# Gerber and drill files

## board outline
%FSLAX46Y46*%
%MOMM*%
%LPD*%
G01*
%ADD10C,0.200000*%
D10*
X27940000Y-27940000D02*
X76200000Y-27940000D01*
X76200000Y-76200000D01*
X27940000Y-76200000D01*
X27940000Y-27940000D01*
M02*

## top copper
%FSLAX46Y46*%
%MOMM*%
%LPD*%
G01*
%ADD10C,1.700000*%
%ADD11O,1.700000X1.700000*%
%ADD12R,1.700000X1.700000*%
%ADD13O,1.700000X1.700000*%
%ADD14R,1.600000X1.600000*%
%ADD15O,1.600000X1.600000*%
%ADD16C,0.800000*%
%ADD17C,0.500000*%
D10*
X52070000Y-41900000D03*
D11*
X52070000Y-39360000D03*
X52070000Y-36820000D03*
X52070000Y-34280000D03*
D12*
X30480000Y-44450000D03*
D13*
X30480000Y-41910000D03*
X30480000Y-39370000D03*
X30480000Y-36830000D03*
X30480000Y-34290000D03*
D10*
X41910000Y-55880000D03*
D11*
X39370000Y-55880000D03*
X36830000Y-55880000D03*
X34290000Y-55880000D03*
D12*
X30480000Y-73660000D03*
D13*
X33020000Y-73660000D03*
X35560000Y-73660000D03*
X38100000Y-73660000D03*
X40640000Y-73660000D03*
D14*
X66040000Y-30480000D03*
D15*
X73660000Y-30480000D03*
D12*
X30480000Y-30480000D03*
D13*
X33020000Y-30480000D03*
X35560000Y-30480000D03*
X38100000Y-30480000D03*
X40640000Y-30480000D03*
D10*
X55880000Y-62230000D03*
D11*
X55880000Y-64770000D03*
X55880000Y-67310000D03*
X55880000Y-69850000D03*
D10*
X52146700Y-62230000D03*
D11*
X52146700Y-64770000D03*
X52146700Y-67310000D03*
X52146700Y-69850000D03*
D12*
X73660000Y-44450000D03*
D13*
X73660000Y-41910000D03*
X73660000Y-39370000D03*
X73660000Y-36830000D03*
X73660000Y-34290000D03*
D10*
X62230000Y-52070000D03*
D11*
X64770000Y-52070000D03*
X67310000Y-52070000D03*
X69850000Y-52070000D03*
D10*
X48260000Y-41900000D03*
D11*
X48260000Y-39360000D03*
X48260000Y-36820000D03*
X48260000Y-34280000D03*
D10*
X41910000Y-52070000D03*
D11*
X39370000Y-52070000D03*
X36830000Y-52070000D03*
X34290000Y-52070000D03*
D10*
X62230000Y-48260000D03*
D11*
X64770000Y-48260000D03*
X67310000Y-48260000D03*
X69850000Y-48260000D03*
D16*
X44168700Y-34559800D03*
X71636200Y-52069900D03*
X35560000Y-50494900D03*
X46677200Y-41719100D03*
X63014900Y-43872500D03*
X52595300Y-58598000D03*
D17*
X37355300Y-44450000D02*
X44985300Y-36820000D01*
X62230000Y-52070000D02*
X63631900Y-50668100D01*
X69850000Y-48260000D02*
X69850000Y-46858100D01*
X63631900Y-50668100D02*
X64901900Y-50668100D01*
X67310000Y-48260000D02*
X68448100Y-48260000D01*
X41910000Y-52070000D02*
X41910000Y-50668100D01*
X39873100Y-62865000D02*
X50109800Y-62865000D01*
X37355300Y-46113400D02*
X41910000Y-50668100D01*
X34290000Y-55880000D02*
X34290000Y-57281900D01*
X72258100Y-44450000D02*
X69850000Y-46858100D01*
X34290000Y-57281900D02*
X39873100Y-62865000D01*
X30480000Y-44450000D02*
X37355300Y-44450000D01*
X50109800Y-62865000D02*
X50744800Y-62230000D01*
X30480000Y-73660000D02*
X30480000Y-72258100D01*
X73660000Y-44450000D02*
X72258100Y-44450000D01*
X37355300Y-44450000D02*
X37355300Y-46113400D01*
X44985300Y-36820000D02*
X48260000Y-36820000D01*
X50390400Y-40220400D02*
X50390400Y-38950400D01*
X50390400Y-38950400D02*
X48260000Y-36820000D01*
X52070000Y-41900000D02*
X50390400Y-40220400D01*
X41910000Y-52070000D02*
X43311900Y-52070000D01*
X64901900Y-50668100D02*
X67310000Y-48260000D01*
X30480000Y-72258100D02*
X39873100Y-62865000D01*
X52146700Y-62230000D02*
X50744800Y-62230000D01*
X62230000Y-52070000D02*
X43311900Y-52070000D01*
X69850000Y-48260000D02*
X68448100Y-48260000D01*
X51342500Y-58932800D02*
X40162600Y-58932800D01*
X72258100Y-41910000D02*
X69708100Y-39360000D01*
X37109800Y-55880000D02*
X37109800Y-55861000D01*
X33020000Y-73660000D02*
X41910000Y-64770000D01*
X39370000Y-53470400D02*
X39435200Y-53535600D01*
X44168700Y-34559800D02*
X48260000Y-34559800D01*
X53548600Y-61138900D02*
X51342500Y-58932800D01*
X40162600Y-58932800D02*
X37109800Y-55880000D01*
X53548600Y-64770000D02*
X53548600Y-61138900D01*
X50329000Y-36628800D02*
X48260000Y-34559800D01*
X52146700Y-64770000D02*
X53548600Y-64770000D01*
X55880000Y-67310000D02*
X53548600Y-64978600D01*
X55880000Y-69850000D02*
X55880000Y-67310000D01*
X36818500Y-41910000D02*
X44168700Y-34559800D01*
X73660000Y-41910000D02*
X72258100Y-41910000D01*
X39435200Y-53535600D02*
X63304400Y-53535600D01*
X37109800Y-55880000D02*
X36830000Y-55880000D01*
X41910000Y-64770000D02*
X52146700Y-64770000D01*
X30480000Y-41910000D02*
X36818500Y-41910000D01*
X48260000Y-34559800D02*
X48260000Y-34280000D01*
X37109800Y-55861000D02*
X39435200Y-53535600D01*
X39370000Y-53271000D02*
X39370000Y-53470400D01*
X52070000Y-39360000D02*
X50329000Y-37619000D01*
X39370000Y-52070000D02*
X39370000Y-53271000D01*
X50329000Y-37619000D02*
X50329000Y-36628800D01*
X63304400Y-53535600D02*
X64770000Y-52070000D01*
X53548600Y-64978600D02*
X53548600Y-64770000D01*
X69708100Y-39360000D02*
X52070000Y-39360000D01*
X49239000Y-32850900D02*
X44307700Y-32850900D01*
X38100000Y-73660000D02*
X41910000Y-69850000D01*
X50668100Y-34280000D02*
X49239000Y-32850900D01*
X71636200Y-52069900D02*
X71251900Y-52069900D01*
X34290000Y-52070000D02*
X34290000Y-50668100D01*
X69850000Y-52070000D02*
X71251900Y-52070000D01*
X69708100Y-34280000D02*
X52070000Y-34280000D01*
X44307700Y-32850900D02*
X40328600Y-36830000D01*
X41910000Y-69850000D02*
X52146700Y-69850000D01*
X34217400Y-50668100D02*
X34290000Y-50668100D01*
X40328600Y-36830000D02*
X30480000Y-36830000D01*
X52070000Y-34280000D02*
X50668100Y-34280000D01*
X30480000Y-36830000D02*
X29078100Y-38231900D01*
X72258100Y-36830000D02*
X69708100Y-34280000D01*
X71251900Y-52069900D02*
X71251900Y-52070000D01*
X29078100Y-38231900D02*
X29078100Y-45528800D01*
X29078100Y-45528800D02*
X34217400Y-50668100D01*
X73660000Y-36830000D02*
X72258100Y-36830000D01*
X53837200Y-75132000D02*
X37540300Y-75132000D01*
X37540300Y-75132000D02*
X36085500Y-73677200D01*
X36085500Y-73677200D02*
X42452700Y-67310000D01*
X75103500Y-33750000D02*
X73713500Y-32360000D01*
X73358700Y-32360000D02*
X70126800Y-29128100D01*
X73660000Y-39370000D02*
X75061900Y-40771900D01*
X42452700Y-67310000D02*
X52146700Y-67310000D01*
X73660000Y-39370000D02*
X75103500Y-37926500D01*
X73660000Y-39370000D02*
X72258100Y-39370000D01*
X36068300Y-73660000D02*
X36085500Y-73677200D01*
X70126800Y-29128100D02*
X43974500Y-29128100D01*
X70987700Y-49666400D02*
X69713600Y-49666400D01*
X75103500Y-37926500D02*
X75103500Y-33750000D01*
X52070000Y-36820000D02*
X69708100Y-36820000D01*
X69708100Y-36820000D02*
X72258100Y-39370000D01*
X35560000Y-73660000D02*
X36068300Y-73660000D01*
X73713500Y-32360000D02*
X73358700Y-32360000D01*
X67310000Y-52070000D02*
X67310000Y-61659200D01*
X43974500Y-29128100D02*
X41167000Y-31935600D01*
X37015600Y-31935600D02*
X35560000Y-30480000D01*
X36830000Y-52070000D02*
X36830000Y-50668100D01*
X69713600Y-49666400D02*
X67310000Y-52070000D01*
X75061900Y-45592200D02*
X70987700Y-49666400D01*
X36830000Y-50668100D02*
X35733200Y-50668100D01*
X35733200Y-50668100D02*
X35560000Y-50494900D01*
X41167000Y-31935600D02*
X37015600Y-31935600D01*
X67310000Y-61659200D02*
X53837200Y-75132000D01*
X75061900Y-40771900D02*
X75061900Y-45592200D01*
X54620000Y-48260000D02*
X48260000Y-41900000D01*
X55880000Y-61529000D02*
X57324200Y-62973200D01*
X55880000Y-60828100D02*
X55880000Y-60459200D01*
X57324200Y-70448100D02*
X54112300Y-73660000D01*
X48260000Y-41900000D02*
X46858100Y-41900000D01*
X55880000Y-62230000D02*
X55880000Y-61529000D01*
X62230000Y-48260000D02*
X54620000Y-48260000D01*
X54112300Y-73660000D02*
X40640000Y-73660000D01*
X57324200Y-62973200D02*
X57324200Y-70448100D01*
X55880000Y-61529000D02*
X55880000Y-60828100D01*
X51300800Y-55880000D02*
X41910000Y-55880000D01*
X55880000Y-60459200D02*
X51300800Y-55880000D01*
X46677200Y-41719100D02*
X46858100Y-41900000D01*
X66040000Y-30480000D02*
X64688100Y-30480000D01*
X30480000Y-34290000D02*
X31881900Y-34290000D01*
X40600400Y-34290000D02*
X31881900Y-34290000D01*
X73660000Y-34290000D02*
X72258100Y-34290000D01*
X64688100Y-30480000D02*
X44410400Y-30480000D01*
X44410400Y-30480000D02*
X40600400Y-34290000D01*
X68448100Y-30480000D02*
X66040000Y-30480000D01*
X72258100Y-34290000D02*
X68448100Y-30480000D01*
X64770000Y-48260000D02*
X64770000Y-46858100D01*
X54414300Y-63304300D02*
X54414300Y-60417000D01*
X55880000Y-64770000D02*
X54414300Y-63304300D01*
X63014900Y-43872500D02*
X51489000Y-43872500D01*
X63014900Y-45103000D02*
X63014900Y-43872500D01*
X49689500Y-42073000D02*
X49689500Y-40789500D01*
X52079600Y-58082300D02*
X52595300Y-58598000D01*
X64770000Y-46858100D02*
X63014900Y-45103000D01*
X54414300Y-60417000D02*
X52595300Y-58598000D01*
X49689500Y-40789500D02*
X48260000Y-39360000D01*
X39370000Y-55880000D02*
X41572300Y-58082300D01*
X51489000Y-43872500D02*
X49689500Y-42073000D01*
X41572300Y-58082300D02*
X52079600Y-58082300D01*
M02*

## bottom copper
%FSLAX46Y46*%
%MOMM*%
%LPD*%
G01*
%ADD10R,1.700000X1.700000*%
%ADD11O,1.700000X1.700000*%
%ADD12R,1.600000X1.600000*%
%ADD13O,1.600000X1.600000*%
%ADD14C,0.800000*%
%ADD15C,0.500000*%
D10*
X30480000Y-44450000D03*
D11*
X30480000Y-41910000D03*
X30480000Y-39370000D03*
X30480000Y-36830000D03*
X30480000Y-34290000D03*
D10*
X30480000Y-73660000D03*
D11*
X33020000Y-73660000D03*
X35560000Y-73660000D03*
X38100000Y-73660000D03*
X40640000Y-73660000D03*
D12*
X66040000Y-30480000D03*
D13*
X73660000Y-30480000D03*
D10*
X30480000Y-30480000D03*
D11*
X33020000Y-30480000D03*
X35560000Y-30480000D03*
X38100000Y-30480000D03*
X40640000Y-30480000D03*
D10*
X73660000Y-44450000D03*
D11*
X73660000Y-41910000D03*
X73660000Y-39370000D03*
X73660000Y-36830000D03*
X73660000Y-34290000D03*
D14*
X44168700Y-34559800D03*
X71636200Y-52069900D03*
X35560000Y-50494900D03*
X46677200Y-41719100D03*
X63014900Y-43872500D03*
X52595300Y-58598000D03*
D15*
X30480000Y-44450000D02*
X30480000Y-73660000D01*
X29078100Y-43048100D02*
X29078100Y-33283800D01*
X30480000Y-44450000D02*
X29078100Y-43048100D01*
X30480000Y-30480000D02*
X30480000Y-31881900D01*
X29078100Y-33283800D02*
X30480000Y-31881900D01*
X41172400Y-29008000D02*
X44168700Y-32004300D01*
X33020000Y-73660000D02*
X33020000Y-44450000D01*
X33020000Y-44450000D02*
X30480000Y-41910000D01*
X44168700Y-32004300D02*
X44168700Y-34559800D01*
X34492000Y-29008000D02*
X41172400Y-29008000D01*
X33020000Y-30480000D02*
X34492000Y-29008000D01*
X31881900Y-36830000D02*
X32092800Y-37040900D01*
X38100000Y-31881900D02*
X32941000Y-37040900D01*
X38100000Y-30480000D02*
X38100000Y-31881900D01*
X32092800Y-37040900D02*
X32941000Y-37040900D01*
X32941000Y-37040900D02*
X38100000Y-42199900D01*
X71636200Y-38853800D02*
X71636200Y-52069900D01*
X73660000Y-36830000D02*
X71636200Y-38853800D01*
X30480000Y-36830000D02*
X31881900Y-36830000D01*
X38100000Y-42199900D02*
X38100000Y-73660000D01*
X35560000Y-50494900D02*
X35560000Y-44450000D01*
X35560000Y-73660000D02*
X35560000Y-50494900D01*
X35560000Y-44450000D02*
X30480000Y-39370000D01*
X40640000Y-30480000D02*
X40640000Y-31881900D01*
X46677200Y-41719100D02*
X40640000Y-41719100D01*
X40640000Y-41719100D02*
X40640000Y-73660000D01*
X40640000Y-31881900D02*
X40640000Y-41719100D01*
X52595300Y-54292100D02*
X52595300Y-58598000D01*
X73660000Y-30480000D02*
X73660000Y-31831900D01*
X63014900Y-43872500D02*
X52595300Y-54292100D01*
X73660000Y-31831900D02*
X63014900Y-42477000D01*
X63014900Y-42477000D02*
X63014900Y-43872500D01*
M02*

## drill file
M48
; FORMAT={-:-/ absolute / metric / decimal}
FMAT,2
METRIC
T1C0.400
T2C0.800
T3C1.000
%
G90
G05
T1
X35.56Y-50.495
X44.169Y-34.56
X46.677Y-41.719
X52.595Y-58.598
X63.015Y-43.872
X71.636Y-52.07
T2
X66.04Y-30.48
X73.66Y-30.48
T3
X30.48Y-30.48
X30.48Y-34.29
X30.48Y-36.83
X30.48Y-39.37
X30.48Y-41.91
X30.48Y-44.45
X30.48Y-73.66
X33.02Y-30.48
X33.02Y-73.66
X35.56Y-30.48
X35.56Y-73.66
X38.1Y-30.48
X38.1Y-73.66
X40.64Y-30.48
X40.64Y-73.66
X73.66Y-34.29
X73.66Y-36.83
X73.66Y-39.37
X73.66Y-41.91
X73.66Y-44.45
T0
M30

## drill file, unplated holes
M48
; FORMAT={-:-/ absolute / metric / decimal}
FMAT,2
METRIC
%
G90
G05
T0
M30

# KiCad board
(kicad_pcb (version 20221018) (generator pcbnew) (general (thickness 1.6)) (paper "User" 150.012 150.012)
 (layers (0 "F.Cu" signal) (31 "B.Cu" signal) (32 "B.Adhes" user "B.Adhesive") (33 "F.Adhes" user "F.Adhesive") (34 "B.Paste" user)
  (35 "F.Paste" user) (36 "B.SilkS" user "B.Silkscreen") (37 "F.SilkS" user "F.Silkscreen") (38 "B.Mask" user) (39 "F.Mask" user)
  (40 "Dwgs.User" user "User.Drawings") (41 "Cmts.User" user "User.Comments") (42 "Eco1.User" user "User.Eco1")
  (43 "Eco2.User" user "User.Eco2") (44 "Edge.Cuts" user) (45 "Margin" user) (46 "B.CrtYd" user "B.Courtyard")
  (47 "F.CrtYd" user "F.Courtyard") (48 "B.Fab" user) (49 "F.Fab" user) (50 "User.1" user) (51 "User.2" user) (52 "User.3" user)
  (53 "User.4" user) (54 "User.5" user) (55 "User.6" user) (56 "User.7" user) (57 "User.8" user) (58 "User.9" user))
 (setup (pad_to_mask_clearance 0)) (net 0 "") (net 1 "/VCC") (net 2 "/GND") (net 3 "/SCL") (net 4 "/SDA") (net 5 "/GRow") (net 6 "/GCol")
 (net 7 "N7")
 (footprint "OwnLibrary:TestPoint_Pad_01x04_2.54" (layer "F.Cu") (at 52.07 41.9 180)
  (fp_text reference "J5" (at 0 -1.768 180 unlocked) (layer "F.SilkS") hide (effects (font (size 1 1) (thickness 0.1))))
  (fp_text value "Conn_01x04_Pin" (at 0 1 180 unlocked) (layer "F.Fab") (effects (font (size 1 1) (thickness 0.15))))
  (pad "1" smd circle (at 0 0 180) (size 1.7 1.7) (layers "F.Cu" "F.Paste" "F.Mask") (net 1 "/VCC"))
  (pad "2" smd oval (at 0 2.54 180) (size 1.7 1.7) (layers "F.Cu" "F.Paste" "F.Mask") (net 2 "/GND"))
  (pad "3" smd oval (at 0 5.08 180) (size 1.7 1.7) (layers "F.Cu" "F.Paste" "F.Mask") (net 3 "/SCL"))
  (pad "4" smd oval (at 0 7.62 180) (size 1.7 1.7) (layers "F.Cu" "F.Paste" "F.Mask") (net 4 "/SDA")))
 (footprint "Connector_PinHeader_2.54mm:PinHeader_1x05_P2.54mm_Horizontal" (layer "F.Cu") (at 30.48 44.45 180)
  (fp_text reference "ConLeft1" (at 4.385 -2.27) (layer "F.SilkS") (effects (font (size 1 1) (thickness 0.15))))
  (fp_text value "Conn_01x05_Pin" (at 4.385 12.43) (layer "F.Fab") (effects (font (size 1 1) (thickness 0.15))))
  (pad "1" thru_hole rect (at 0 0 180) (size 1.7 1.7) (drill 1) (layers "*.Cu" "*.Mask") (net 1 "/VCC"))
  (pad "2" thru_hole oval (at 0 2.54 180) (size 1.7 1.7) (drill 1) (layers "*.Cu" "*.Mask") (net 2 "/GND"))
  (pad "3" thru_hole oval (at 0 5.08 180) (size 1.7 1.7) (drill 1) (layers "*.Cu" "*.Mask") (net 3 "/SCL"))
  (pad "4" thru_hole oval (at 0 7.62 180) (size 1.7 1.7) (drill 1) (layers "*.Cu" "*.Mask") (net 4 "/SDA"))
  (pad "5" thru_hole oval (at 0 10.16 180) (size 1.7 1.7) (drill 1) (layers "*.Cu" "*.Mask") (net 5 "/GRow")))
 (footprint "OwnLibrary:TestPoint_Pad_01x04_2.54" (layer "F.Cu") (at 41.91 55.88 -90)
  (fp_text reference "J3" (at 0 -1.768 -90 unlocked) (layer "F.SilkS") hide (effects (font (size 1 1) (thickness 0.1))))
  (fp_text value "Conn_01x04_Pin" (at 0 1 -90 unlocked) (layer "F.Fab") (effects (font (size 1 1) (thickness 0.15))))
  (pad "1" smd circle (at 0 0 270) (size 1.7 1.7) (layers "F.Cu" "F.Paste" "F.Mask") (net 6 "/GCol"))
  (pad "2" smd oval (at 0 2.54 270) (size 1.7 1.7) (layers "F.Cu" "F.Paste" "F.Mask") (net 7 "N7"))
  (pad "3" smd oval (at 0 5.08 270) (size 1.7 1.7) (layers "F.Cu" "F.Paste" "F.Mask") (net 2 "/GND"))
  (pad "4" smd oval (at 0 7.62 270) (size 1.7 1.7) (layers "F.Cu" "F.Paste" "F.Mask") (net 1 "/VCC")))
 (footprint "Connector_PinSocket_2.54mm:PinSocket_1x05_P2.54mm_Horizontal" (layer "F.Cu") (at 30.48 73.66 90)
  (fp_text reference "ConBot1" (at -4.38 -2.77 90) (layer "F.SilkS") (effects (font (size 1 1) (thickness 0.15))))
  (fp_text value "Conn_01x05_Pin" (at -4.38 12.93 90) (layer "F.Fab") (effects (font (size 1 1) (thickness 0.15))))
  (pad "1" thru_hole rect (at 0 0 90) (size 1.7 1.7) (drill 1) (layers "*.Cu" "*.Mask") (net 1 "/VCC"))
  (pad "2" thru_hole oval (at 0 2.54 90) (size 1.7 1.7) (drill 1) (layers "*.Cu" "*.Mask") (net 2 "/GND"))
  (pad "3" thru_hole oval (at 0 5.08 90) (size 1.7 1.7) (drill 1) (layers "*.Cu" "*.Mask") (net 3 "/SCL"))
  (pad "4" thru_hole oval (at 0 7.62 90) (size 1.7 1.7) (drill 1) (layers "*.Cu" "*.Mask") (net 4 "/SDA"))
  (pad "5" thru_hole oval (at 0 10.16 90) (size 1.7 1.7) (drill 1) (layers "*.Cu" "*.Mask") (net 6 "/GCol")))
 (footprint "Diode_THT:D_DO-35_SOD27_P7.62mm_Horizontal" (layer "F.Cu") (at 66.04 30.48)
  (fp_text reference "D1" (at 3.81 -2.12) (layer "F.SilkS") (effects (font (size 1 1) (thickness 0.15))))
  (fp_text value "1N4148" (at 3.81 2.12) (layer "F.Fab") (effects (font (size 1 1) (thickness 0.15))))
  (pad "1" thru_hole rect (at 0 0) (size 1.6 1.6) (drill 0.8) (layers "*.Cu" "*.Mask") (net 5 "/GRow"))
  (pad "2" thru_hole oval (at 7.62 0) (size 1.6 1.6) (drill 0.8) (layers "*.Cu" "*.Mask") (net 7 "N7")))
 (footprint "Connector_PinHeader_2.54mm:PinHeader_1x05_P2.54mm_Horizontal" (layer "F.Cu") (at 30.48 30.48 90)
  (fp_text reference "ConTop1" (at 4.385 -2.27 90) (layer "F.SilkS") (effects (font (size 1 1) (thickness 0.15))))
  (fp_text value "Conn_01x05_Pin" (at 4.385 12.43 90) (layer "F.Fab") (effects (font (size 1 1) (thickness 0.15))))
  (pad "1" thru_hole rect (at 0 0 90) (size 1.7 1.7) (drill 1) (layers "*.Cu" "*.Mask") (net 1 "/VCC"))
  (pad "2" thru_hole oval (at 0 2.54 90) (size 1.7 1.7) (drill 1) (layers "*.Cu" "*.Mask") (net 2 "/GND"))
  (pad "3" thru_hole oval (at 0 5.08 90) (size 1.7 1.7) (drill 1) (layers "*.Cu" "*.Mask") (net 3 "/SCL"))
  (pad "4" thru_hole oval (at 0 7.62 90) (size 1.7 1.7) (drill 1) (layers "*.Cu" "*.Mask") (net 4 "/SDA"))
  (pad "5" thru_hole oval (at 0 10.16 90) (size 1.7 1.7) (drill 1) (layers "*.Cu" "*.Mask") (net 6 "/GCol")))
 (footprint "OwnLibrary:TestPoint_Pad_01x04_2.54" (layer "F.Cu") (at 55.88 62.23)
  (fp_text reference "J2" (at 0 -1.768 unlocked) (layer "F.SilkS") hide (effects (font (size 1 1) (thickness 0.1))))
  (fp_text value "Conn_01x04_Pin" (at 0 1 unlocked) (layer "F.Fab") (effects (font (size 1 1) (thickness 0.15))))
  (pad "1" smd circle (at 0 0) (size 1.7 1.7) (layers "F.Cu" "F.Paste" "F.Mask") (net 6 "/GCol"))
  (pad "2" smd oval (at 0 2.54) (size 1.7 1.7) (layers "F.Cu" "F.Paste" "F.Mask") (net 7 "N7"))
  (pad "3" smd oval (at 0 5.08) (size 1.7 1.7) (layers "F.Cu" "F.Paste" "F.Mask") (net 2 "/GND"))
  (pad "4" smd oval (at 0 7.62) (size 1.7 1.7) (layers "F.Cu" "F.Paste" "F.Mask") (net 2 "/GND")))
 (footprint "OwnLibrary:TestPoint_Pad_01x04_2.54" (layer "F.Cu") (at 52.1467 62.23)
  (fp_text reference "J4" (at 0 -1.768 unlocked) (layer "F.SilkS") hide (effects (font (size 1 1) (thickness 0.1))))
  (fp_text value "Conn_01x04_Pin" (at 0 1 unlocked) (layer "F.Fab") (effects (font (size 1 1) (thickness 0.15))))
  (pad "1" smd circle (at 0 0) (size 1.7 1.7) (layers "F.Cu" "F.Paste" "F.Mask") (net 1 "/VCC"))
  (pad "2" smd oval (at 0 2.54) (size 1.7 1.7) (layers "F.Cu" "F.Paste" "F.Mask") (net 2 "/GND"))
  (pad "3" smd oval (at 0 5.08) (size 1.7 1.7) (layers "F.Cu" "F.Paste" "F.Mask") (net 3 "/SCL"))
  (pad "4" smd oval (at 0 7.62) (size 1.7 1.7) (layers "F.Cu" "F.Paste" "F.Mask") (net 4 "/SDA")))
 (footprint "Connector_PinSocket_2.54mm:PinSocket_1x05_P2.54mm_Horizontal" (layer "F.Cu") (at 73.66 44.45 180)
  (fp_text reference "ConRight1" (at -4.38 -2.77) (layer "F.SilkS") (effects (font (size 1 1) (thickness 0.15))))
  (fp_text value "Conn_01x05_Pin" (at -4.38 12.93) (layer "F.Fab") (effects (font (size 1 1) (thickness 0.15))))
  (pad "1" thru_hole rect (at 0 0 180) (size 1.7 1.7) (drill 1) (layers "*.Cu" "*.Mask") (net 1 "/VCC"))
  (pad "2" thru_hole oval (at 0 2.54 180) (size 1.7 1.7) (drill 1) (layers "*.Cu" "*.Mask") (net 2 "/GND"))
  (pad "3" thru_hole oval (at 0 5.08 180) (size 1.7 1.7) (drill 1) (layers "*.Cu" "*.Mask") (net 3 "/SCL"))
  (pad "4" thru_hole oval (at 0 7.62 180) (size 1.7 1.7) (drill 1) (layers "*.Cu" "*.Mask") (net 4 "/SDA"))
  (pad "5" thru_hole oval (at 0 10.16 180) (size 1.7 1.7) (drill 1) (layers "*.Cu" "*.Mask") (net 5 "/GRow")))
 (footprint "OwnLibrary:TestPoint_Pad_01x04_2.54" (layer "F.Cu") (at 62.23 52.07 90)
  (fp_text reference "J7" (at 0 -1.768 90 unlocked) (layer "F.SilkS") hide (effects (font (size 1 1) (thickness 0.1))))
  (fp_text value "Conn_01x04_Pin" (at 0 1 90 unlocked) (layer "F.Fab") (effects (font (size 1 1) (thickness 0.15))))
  (pad "1" smd circle (at 0 0 90) (size 1.7 1.7) (layers "F.Cu" "F.Paste" "F.Mask") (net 1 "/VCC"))
  (pad "2" smd oval (at 0 2.54 90) (size 1.7 1.7) (layers "F.Cu" "F.Paste" "F.Mask") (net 2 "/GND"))
  (pad "3" smd oval (at 0 5.08 90) (size 1.7 1.7) (layers "F.Cu" "F.Paste" "F.Mask") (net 3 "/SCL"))
  (pad "4" smd oval (at 0 7.62 90) (size 1.7 1.7) (layers "F.Cu" "F.Paste" "F.Mask") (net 4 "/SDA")))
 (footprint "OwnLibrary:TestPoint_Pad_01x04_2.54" (layer "F.Cu") (at 48.26 41.9 180)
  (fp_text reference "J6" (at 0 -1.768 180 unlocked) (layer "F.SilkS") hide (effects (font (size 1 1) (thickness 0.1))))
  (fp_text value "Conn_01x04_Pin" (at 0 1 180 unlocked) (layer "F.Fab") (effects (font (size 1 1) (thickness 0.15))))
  (pad "1" smd circle (at 0 0 180) (size 1.7 1.7) (layers "F.Cu" "F.Paste" "F.Mask") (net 6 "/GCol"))
  (pad "2" smd oval (at 0 2.54 180) (size 1.7 1.7) (layers "F.Cu" "F.Paste" "F.Mask") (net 7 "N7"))
  (pad "3" smd oval (at 0 5.08 180) (size 1.7 1.7) (layers "F.Cu" "F.Paste" "F.Mask") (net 1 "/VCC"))
  (pad "4" smd oval (at 0 7.62 180) (size 1.7 1.7) (layers "F.Cu" "F.Paste" "F.Mask") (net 2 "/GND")))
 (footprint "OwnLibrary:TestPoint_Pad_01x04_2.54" (layer "F.Cu") (at 41.91 52.07 -90)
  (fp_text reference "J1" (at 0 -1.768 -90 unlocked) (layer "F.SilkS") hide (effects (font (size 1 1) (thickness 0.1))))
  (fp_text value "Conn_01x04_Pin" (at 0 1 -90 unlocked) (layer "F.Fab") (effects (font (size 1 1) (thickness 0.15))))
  (pad "1" smd circle (at 0 0 270) (size 1.7 1.7) (layers "F.Cu" "F.Paste" "F.Mask") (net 1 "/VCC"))
  (pad "2" smd oval (at 0 2.54 270) (size 1.7 1.7) (layers "F.Cu" "F.Paste" "F.Mask") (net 2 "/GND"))
  (pad "3" smd oval (at 0 5.08 270) (size 1.7 1.7) (layers "F.Cu" "F.Paste" "F.Mask") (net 3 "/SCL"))
  (pad "4" smd oval (at 0 7.62 270) (size 1.7 1.7) (layers "F.Cu" "F.Paste" "F.Mask") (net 4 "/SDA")))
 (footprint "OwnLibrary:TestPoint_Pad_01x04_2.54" (layer "F.Cu") (at 62.23 48.26 90)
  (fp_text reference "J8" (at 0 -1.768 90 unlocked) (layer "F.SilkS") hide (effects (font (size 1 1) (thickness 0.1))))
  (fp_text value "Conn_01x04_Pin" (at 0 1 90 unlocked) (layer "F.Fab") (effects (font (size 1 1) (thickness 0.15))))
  (pad "1" smd circle (at 0 0 90) (size 1.7 1.7) (layers "F.Cu" "F.Paste" "F.Mask") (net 6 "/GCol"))
  (pad "2" smd oval (at 0 2.54 90) (size 1.7 1.7) (layers "F.Cu" "F.Paste" "F.Mask") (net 7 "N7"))
  (pad "3" smd oval (at 0 5.08 90) (size 1.7 1.7) (layers "F.Cu" "F.Paste" "F.Mask") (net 1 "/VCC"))
  (pad "4" smd oval (at 0 7.62 90) (size 1.7 1.7) (layers "F.Cu" "F.Paste" "F.Mask") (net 1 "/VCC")))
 (gr_rect (start 27.94 27.94) (end 76.2 76.2) (stroke (width 0.2) (type default)) (fill none) (layer "Edge.Cuts"))
 (segment (start 37.3553 44.45) (end 44.9853 36.82) (width 0.5) (layer "F.Cu") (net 1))
 (segment (start 62.23 52.07) (end 63.6319 50.6681) (width 0.5) (layer "F.Cu") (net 1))
 (segment (start 69.85 48.26) (end 69.85 46.8581) (width 0.5) (layer "F.Cu") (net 1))
 (segment (start 63.6319 50.6681) (end 64.9019 50.6681) (width 0.5) (layer "F.Cu") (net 1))
 (segment (start 67.31 48.26) (end 68.4481 48.26) (width 0.5) (layer "F.Cu") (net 1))
 (segment (start 41.91 52.07) (end 41.91 50.6681) (width 0.5) (layer "F.Cu") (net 1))
 (segment (start 39.8731 62.865) (end 50.1098 62.865) (width 0.5) (layer "F.Cu") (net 1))
 (segment (start 37.3553 46.1134) (end 41.91 50.6681) (width 0.5) (layer "F.Cu") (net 1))
 (segment (start 34.29 55.88) (end 34.29 57.2819) (width 0.5) (layer "F.Cu") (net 1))
 (segment (start 72.2581 44.45) (end 69.85 46.8581) (width 0.5) (layer "F.Cu") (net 1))
 (segment (start 34.29 57.2819) (end 39.8731 62.865) (width 0.5) (layer "F.Cu") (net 1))
 (segment (start 30.48 44.45) (end 37.3553 44.45) (width 0.5) (layer "F.Cu") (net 1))
 (segment (start 50.1098 62.865) (end 50.7448 62.23) (width 0.5) (layer "F.Cu") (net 1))
 (segment (start 30.48 73.66) (end 30.48 72.2581) (width 0.5) (layer "F.Cu") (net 1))
 (segment (start 73.66 44.45) (end 72.2581 44.45) (width 0.5) (layer "F.Cu") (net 1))
 (segment (start 37.3553 44.45) (end 37.3553 46.1134) (width 0.5) (layer "F.Cu") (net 1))
 (segment (start 44.9853 36.82) (end 48.26 36.82) (width 0.5) (layer "F.Cu") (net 1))
 (segment (start 50.3904 40.2204) (end 50.3904 38.9504) (width 0.5) (layer "F.Cu") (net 1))
 (segment (start 50.3904 38.9504) (end 48.26 36.82) (width 0.5) (layer "F.Cu") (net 1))
 (segment (start 52.07 41.9) (end 50.3904 40.2204) (width 0.5) (layer "F.Cu") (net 1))
 (segment (start 41.91 52.07) (end 43.3119 52.07) (width 0.5) (layer "F.Cu") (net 1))
 (segment (start 64.9019 50.6681) (end 67.31 48.26) (width 0.5) (layer "F.Cu") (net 1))
 (segment (start 30.48 72.2581) (end 39.8731 62.865) (width 0.5) (layer "F.Cu") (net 1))
 (segment (start 52.1467 62.23) (end 50.7448 62.23) (width 0.5) (layer "F.Cu") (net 1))
 (segment (start 62.23 52.07) (end 43.3119 52.07) (width 0.5) (layer "F.Cu") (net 1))
 (segment (start 69.85 48.26) (end 68.4481 48.26) (width 0.5) (layer "F.Cu") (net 1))
 (segment (start 30.48 44.45) (end 30.48 73.66) (width 0.5) (layer "B.Cu") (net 1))
 (segment (start 29.0781 43.0481) (end 29.0781 33.2838) (width 0.5) (layer "B.Cu") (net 1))
 (segment (start 30.48 44.45) (end 29.0781 43.0481) (width 0.5) (layer "B.Cu") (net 1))
 (segment (start 30.48 30.48) (end 30.48 31.8819) (width 0.5) (layer "B.Cu") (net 1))
 (segment (start 29.0781 33.2838) (end 30.48 31.8819) (width 0.5) (layer "B.Cu") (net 1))
 (segment (start 51.3425 58.9328) (end 40.1626 58.9328) (width 0.5) (layer "F.Cu") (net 2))
 (segment (start 72.2581 41.91) (end 69.7081 39.36) (width 0.5) (layer "F.Cu") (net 2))
 (segment (start 37.1098 55.88) (end 37.1098 55.861) (width 0.5) (layer "F.Cu") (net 2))
 (segment (start 33.02 73.66) (end 41.91 64.77) (width 0.5) (layer "F.Cu") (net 2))
 (segment (start 39.37 53.4704) (end 39.4352 53.5356) (width 0.5) (layer "F.Cu") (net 2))
 (segment (start 44.1687 34.5598) (end 48.26 34.5598) (width 0.5) (layer "F.Cu") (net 2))
 (segment (start 53.5486 61.1389) (end 51.3425 58.9328) (width 0.5) (layer "F.Cu") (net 2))
 (segment (start 40.1626 58.9328) (end 37.1098 55.88) (width 0.5) (layer "F.Cu") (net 2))
 (segment (start 53.5486 64.77) (end 53.5486 61.1389) (width 0.5) (layer "F.Cu") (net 2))
 (segment (start 50.329 36.6288) (end 48.26 34.5598) (width 0.5) (layer "F.Cu") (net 2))
 (segment (start 52.1467 64.77) (end 53.5486 64.77) (width 0.5) (layer "F.Cu") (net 2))
 (segment (start 55.88 67.31) (end 53.5486 64.9786) (width 0.5) (layer "F.Cu") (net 2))
 (segment (start 55.88 69.85) (end 55.88 67.31) (width 0.5) (layer "F.Cu") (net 2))
 (segment (start 36.8185 41.91) (end 44.1687 34.5598) (width 0.5) (layer "F.Cu") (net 2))
 (segment (start 73.66 41.91) (end 72.2581 41.91) (width 0.5) (layer "F.Cu") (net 2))
 (segment (start 39.4352 53.5356) (end 63.3044 53.5356) (width 0.5) (layer "F.Cu") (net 2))
 (segment (start 37.1098 55.88) (end 36.83 55.88) (width 0.5) (layer "F.Cu") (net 2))
 (segment (start 41.91 64.77) (end 52.1467 64.77) (width 0.5) (layer "F.Cu") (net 2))
 (segment (start 30.48 41.91) (end 36.8185 41.91) (width 0.5) (layer "F.Cu") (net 2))
 (segment (start 48.26 34.5598) (end 48.26 34.28) (width 0.5) (layer "F.Cu") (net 2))
 (segment (start 37.1098 55.861) (end 39.4352 53.5356) (width 0.5) (layer "F.Cu") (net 2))
 (segment (start 39.37 53.271) (end 39.37 53.4704) (width 0.5) (layer "F.Cu") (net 2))
 (segment (start 52.07 39.36) (end 50.329 37.619) (width 0.5) (layer "F.Cu") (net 2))
 (segment (start 39.37 52.07) (end 39.37 53.271) (width 0.5) (layer "F.Cu") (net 2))
 (segment (start 50.329 37.619) (end 50.329 36.6288) (width 0.5) (layer "F.Cu") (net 2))
 (segment (start 63.3044 53.5356) (end 64.77 52.07) (width 0.5) (layer "F.Cu") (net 2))
 (segment (start 53.5486 64.9786) (end 53.5486 64.77) (width 0.5) (layer "F.Cu") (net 2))
 (segment (start 69.7081 39.36) (end 52.07 39.36) (width 0.5) (layer "F.Cu") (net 2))
 (via (at 44.1687 34.5598) (size 0.8) (drill 0.4) (layers "F.Cu" "B.Cu") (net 2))
 (segment (start 41.1724 29.008) (end 44.1687 32.0043) (width 0.5) (layer "B.Cu") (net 2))
 (segment (start 33.02 73.66) (end 33.02 44.45) (width 0.5) (layer "B.Cu") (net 2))
 (segment (start 33.02 44.45) (end 30.48 41.91) (width 0.5) (layer "B.Cu") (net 2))
 (segment (start 44.1687 32.0043) (end 44.1687 34.5598) (width 0.5) (layer "B.Cu") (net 2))
 (segment (start 34.492 29.008) (end 41.1724 29.008) (width 0.5) (layer "B.Cu") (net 2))
 (segment (start 33.02 30.48) (end 34.492 29.008) (width 0.5) (layer "B.Cu") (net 2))
 (segment (start 49.239 32.8509) (end 44.3077 32.8509) (width 0.5) (layer "F.Cu") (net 4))
 (segment (start 38.1 73.66) (end 41.91 69.85) (width 0.5) (layer "F.Cu") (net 4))
 (segment (start 50.6681 34.28) (end 49.239 32.8509) (width 0.5) (layer "F.Cu") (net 4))
 (segment (start 71.6362 52.0699) (end 71.2519 52.0699) (width 0.5) (layer "F.Cu") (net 4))
 (segment (start 34.29 52.07) (end 34.29 50.6681) (width 0.5) (layer "F.Cu") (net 4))
 (segment (start 69.85 52.07) (end 71.2519 52.07) (width 0.5) (layer "F.Cu") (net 4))
 (segment (start 69.7081 34.28) (end 52.07 34.28) (width 0.5) (layer "F.Cu") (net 4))
 (segment (start 44.3077 32.8509) (end 40.3286 36.83) (width 0.5) (layer "F.Cu") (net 4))
 (segment (start 41.91 69.85) (end 52.1467 69.85) (width 0.5) (layer "F.Cu") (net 4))
 (segment (start 34.2174 50.6681) (end 34.29 50.6681) (width 0.5) (layer "F.Cu") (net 4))
 (segment (start 40.3286 36.83) (end 30.48 36.83) (width 0.5) (layer "F.Cu") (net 4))
 (segment (start 52.07 34.28) (end 50.6681 34.28) (width 0.5) (layer "F.Cu") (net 4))
 (segment (start 30.48 36.83) (end 29.0781 38.2319) (width 0.5) (layer "F.Cu") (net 4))
 (segment (start 72.2581 36.83) (end 69.7081 34.28) (width 0.5) (layer "F.Cu") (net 4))
 (segment (start 71.2519 52.0699) (end 71.2519 52.07) (width 0.5) (layer "F.Cu") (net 4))
 (segment (start 29.0781 38.2319) (end 29.0781 45.5288) (width 0.5) (layer "F.Cu") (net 4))
 (segment (start 29.0781 45.5288) (end 34.2174 50.6681) (width 0.5) (layer "F.Cu") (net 4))
 (segment (start 73.66 36.83) (end 72.2581 36.83) (width 0.5) (layer "F.Cu") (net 4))
 (via (at 71.6362 52.0699) (size 0.8) (drill 0.4) (layers "F.Cu" "B.Cu") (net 4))
 (segment (start 31.8819 36.83) (end 32.0928 37.0409) (width 0.5) (layer "B.Cu") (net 4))
 (segment (start 38.1 31.8819) (end 32.941 37.0409) (width 0.5) (layer "B.Cu") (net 4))
 (segment (start 38.1 30.48) (end 38.1 31.8819) (width 0.5) (layer "B.Cu") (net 4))
 (segment (start 32.0928 37.0409) (end 32.941 37.0409) (width 0.5) (layer "B.Cu") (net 4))
 (segment (start 32.941 37.0409) (end 38.1 42.1999) (width 0.5) (layer "B.Cu") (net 4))
 (segment (start 71.6362 38.8538) (end 71.6362 52.0699) (width 0.5) (layer "B.Cu") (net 4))
 (segment (start 73.66 36.83) (end 71.6362 38.8538) (width 0.5) (layer "B.Cu") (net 4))
 (segment (start 30.48 36.83) (end 31.8819 36.83) (width 0.5) (layer "B.Cu") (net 4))
 (segment (start 38.1 42.1999) (end 38.1 73.66) (width 0.5) (layer "B.Cu") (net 4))
 (segment (start 53.8372 75.132) (end 37.5403 75.132) (width 0.5) (layer "F.Cu") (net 3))
 (segment (start 37.5403 75.132) (end 36.0855 73.6772) (width 0.5) (layer "F.Cu") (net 3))
 (segment (start 36.0855 73.6772) (end 42.4527 67.31) (width 0.5) (layer "F.Cu") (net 3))
 (segment (start 75.1035 33.75) (end 73.7135 32.36) (width 0.5) (layer "F.Cu") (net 3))
 (segment (start 73.3587 32.36) (end 70.1268 29.1281) (width 0.5) (layer "F.Cu") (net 3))
 (segment (start 73.66 39.37) (end 75.0619 40.7719) (width 0.5) (layer "F.Cu") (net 3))
 (segment (start 42.4527 67.31) (end 52.1467 67.31) (width 0.5) (layer "F.Cu") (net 3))
 (segment (start 73.66 39.37) (end 75.1035 37.9265) (width 0.5) (layer "F.Cu") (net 3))
 (segment (start 73.66 39.37) (end 72.2581 39.37) (width 0.5) (layer "F.Cu") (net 3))
 (segment (start 36.0683 73.66) (end 36.0855 73.6772) (width 0.5) (layer "F.Cu") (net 3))
 (segment (start 70.1268 29.1281) (end 43.9745 29.1281) (width 0.5) (layer "F.Cu") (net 3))
 (segment (start 70.9877 49.6664) (end 69.7136 49.6664) (width 0.5) (layer "F.Cu") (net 3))
 (segment (start 75.1035 37.9265) (end 75.1035 33.75) (width 0.5) (layer "F.Cu") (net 3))
 (segment (start 52.07 36.82) (end 69.7081 36.82) (width 0.5) (layer "F.Cu") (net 3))
 (segment (start 69.7081 36.82) (end 72.2581 39.37) (width 0.5) (layer "F.Cu") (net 3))
 (segment (start 35.56 73.66) (end 36.0683 73.66) (width 0.5) (layer "F.Cu") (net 3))
 (segment (start 73.7135 32.36) (end 73.3587 32.36) (width 0.5) (layer "F.Cu") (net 3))
 (segment (start 67.31 52.07) (end 67.31 61.6592) (width 0.5) (layer "F.Cu") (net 3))
 (segment (start 43.9745 29.1281) (end 41.167 31.9356) (width 0.5) (layer "F.Cu") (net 3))
 (segment (start 37.0156 31.9356) (end 35.56 30.48) (width 0.5) (layer "F.Cu") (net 3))
 (segment (start 36.83 52.07) (end 36.83 50.6681) (width 0.5) (layer "F.Cu") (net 3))
 (segment (start 69.7136 49.6664) (end 67.31 52.07) (width 0.5) (layer "F.Cu") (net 3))
 (segment (start 75.0619 45.5922) (end 70.9877 49.6664) (width 0.5) (layer "F.Cu") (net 3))
 (segment (start 36.83 50.6681) (end 35.7332 50.6681) (width 0.5) (layer "F.Cu") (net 3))
 (segment (start 35.7332 50.6681) (end 35.56 50.4949) (width 0.5) (layer "F.Cu") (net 3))
 (segment (start 41.167 31.9356) (end 37.0156 31.9356) (width 0.5) (layer "F.Cu") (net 3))
 (segment (start 67.31 61.6592) (end 53.8372 75.132) (width 0.5) (layer "F.Cu") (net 3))
 (segment (start 75.0619 40.7719) (end 75.0619 45.5922) (width 0.5) (layer "F.Cu") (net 3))
 (via (at 35.56 50.4949) (size 0.8) (drill 0.4) (layers "F.Cu" "B.Cu") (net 3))
 (segment (start 35.56 50.4949) (end 35.56 44.45) (width 0.5) (layer "B.Cu") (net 3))
 (segment (start 35.56 73.66) (end 35.56 50.4949) (width 0.5) (layer "B.Cu") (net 3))
 (segment (start 35.56 44.45) (end 30.48 39.37) (width 0.5) (layer "B.Cu") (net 3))
 (segment (start 54.62 48.26) (end 48.26 41.9) (width 0.5) (layer "F.Cu") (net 6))
 (segment (start 55.88 61.529) (end 57.3242 62.9732) (width 0.5) (layer "F.Cu") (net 6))
 (segment (start 55.88 60.8281) (end 55.88 60.4592) (width 0.5) (layer "F.Cu") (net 6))
 (segment (start 57.3242 70.4481) (end 54.1123 73.66) (width 0.5) (layer "F.Cu") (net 6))
 (segment (start 48.26 41.9) (end 46.8581 41.9) (width 0.5) (layer "F.Cu") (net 6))
 (segment (start 55.88 62.23) (end 55.88 61.529) (width 0.5) (layer "F.Cu") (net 6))
 (segment (start 62.23 48.26) (end 54.62 48.26) (width 0.5) (layer "F.Cu") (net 6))
 (segment (start 54.1123 73.66) (end 40.64 73.66) (width 0.5) (layer "F.Cu") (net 6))
 (segment (start 57.3242 62.9732) (end 57.3242 70.4481) (width 0.5) (layer "F.Cu") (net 6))
 (segment (start 55.88 61.529) (end 55.88 60.8281) (width 0.5) (layer "F.Cu") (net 6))
 (segment (start 51.3008 55.88) (end 41.91 55.88) (width 0.5) (layer "F.Cu") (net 6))
 (segment (start 55.88 60.4592) (end 51.3008 55.88) (width 0.5) (layer "F.Cu") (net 6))
 (segment (start 46.6772 41.7191) (end 46.8581 41.9) (width 0.5) (layer "F.Cu") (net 6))
 (via (at 46.6772 41.7191) (size 0.8) (drill 0.4) (layers "F.Cu" "B.Cu") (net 6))
 (segment (start 40.64 30.48) (end 40.64 31.8819) (width 0.5) (layer "B.Cu") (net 6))
 (segment (start 46.6772 41.7191) (end 40.64 41.7191) (width 0.5) (layer "B.Cu") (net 6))
 (segment (start 40.64 41.7191) (end 40.64 73.66) (width 0.5) (layer "B.Cu") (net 6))
 (segment (start 40.64 31.8819) (end 40.64 41.7191) (width 0.5) (layer "B.Cu") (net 6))
 (segment (start 66.04 30.48) (end 64.6881 30.48) (width 0.5) (layer "F.Cu") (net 5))
 (segment (start 30.48 34.29) (end 31.8819 34.29) (width 0.5) (layer "F.Cu") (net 5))
 (segment (start 40.6004 34.29) (end 31.8819 34.29) (width 0.5) (layer "F.Cu") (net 5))
 (segment (start 73.66 34.29) (end 72.2581 34.29) (width 0.5) (layer "F.Cu") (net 5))
 (segment (start 64.6881 30.48) (end 44.4104 30.48) (width 0.5) (layer "F.Cu") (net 5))
 (segment (start 44.4104 30.48) (end 40.6004 34.29) (width 0.5) (layer "F.Cu") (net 5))
 (segment (start 68.4481 30.48) (end 66.04 30.48) (width 0.5) (layer "F.Cu") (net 5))
 (segment (start 72.2581 34.29) (end 68.4481 30.48) (width 0.5) (layer "F.Cu") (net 5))
 (segment (start 64.77 48.26) (end 64.77 46.8581) (width 0.5) (layer "F.Cu") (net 7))
 (segment (start 54.4143 63.3043) (end 54.4143 60.417) (width 0.5) (layer "F.Cu") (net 7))
 (segment (start 55.88 64.77) (end 54.4143 63.3043) (width 0.5) (layer "F.Cu") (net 7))
 (segment (start 63.0149 43.8725) (end 51.489 43.8725) (width 0.5) (layer "F.Cu") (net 7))
 (segment (start 63.0149 45.103) (end 63.0149 43.8725) (width 0.5) (layer "F.Cu") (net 7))
 (segment (start 49.6895 42.073) (end 49.6895 40.7895) (width 0.5) (layer "F.Cu") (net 7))
 (segment (start 52.0796 58.0823) (end 52.5953 58.598) (width 0.5) (layer "F.Cu") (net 7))
 (segment (start 64.77 46.8581) (end 63.0149 45.103) (width 0.5) (layer "F.Cu") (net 7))
 (segment (start 54.4143 60.417) (end 52.5953 58.598) (width 0.5) (layer "F.Cu") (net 7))
 (segment (start 49.6895 40.7895) (end 48.26 39.36) (width 0.5) (layer "F.Cu") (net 7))
 (segment (start 39.37 55.88) (end 41.5723 58.0823) (width 0.5) (layer "F.Cu") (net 7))
 (segment (start 51.489 43.8725) (end 49.6895 42.073) (width 0.5) (layer "F.Cu") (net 7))
 (segment (start 41.5723 58.0823) (end 52.0796 58.0823) (width 0.5) (layer "F.Cu") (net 7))
 (via (at 63.0149 43.8725) (size 0.8) (drill 0.4) (layers "F.Cu" "B.Cu") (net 7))
 (via (at 52.5953 58.598) (size 0.8) (drill 0.4) (layers "F.Cu" "B.Cu") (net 7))
 (segment (start 52.5953 54.2921) (end 52.5953 58.598) (width 0.5) (layer "B.Cu") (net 7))
 (segment (start 73.66 30.48) (end 73.66 31.8319) (width 0.5) (layer "B.Cu") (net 7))
 (segment (start 63.0149 43.8725) (end 52.5953 54.2921) (width 0.5) (layer "B.Cu") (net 7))
 (segment (start 73.66 31.8319) (end 63.0149 42.477) (width 0.5) (layer "B.Cu") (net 7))
 (segment (start 63.0149 42.477) (end 63.0149 43.8725) (width 0.5) (layer "B.Cu") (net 7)))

